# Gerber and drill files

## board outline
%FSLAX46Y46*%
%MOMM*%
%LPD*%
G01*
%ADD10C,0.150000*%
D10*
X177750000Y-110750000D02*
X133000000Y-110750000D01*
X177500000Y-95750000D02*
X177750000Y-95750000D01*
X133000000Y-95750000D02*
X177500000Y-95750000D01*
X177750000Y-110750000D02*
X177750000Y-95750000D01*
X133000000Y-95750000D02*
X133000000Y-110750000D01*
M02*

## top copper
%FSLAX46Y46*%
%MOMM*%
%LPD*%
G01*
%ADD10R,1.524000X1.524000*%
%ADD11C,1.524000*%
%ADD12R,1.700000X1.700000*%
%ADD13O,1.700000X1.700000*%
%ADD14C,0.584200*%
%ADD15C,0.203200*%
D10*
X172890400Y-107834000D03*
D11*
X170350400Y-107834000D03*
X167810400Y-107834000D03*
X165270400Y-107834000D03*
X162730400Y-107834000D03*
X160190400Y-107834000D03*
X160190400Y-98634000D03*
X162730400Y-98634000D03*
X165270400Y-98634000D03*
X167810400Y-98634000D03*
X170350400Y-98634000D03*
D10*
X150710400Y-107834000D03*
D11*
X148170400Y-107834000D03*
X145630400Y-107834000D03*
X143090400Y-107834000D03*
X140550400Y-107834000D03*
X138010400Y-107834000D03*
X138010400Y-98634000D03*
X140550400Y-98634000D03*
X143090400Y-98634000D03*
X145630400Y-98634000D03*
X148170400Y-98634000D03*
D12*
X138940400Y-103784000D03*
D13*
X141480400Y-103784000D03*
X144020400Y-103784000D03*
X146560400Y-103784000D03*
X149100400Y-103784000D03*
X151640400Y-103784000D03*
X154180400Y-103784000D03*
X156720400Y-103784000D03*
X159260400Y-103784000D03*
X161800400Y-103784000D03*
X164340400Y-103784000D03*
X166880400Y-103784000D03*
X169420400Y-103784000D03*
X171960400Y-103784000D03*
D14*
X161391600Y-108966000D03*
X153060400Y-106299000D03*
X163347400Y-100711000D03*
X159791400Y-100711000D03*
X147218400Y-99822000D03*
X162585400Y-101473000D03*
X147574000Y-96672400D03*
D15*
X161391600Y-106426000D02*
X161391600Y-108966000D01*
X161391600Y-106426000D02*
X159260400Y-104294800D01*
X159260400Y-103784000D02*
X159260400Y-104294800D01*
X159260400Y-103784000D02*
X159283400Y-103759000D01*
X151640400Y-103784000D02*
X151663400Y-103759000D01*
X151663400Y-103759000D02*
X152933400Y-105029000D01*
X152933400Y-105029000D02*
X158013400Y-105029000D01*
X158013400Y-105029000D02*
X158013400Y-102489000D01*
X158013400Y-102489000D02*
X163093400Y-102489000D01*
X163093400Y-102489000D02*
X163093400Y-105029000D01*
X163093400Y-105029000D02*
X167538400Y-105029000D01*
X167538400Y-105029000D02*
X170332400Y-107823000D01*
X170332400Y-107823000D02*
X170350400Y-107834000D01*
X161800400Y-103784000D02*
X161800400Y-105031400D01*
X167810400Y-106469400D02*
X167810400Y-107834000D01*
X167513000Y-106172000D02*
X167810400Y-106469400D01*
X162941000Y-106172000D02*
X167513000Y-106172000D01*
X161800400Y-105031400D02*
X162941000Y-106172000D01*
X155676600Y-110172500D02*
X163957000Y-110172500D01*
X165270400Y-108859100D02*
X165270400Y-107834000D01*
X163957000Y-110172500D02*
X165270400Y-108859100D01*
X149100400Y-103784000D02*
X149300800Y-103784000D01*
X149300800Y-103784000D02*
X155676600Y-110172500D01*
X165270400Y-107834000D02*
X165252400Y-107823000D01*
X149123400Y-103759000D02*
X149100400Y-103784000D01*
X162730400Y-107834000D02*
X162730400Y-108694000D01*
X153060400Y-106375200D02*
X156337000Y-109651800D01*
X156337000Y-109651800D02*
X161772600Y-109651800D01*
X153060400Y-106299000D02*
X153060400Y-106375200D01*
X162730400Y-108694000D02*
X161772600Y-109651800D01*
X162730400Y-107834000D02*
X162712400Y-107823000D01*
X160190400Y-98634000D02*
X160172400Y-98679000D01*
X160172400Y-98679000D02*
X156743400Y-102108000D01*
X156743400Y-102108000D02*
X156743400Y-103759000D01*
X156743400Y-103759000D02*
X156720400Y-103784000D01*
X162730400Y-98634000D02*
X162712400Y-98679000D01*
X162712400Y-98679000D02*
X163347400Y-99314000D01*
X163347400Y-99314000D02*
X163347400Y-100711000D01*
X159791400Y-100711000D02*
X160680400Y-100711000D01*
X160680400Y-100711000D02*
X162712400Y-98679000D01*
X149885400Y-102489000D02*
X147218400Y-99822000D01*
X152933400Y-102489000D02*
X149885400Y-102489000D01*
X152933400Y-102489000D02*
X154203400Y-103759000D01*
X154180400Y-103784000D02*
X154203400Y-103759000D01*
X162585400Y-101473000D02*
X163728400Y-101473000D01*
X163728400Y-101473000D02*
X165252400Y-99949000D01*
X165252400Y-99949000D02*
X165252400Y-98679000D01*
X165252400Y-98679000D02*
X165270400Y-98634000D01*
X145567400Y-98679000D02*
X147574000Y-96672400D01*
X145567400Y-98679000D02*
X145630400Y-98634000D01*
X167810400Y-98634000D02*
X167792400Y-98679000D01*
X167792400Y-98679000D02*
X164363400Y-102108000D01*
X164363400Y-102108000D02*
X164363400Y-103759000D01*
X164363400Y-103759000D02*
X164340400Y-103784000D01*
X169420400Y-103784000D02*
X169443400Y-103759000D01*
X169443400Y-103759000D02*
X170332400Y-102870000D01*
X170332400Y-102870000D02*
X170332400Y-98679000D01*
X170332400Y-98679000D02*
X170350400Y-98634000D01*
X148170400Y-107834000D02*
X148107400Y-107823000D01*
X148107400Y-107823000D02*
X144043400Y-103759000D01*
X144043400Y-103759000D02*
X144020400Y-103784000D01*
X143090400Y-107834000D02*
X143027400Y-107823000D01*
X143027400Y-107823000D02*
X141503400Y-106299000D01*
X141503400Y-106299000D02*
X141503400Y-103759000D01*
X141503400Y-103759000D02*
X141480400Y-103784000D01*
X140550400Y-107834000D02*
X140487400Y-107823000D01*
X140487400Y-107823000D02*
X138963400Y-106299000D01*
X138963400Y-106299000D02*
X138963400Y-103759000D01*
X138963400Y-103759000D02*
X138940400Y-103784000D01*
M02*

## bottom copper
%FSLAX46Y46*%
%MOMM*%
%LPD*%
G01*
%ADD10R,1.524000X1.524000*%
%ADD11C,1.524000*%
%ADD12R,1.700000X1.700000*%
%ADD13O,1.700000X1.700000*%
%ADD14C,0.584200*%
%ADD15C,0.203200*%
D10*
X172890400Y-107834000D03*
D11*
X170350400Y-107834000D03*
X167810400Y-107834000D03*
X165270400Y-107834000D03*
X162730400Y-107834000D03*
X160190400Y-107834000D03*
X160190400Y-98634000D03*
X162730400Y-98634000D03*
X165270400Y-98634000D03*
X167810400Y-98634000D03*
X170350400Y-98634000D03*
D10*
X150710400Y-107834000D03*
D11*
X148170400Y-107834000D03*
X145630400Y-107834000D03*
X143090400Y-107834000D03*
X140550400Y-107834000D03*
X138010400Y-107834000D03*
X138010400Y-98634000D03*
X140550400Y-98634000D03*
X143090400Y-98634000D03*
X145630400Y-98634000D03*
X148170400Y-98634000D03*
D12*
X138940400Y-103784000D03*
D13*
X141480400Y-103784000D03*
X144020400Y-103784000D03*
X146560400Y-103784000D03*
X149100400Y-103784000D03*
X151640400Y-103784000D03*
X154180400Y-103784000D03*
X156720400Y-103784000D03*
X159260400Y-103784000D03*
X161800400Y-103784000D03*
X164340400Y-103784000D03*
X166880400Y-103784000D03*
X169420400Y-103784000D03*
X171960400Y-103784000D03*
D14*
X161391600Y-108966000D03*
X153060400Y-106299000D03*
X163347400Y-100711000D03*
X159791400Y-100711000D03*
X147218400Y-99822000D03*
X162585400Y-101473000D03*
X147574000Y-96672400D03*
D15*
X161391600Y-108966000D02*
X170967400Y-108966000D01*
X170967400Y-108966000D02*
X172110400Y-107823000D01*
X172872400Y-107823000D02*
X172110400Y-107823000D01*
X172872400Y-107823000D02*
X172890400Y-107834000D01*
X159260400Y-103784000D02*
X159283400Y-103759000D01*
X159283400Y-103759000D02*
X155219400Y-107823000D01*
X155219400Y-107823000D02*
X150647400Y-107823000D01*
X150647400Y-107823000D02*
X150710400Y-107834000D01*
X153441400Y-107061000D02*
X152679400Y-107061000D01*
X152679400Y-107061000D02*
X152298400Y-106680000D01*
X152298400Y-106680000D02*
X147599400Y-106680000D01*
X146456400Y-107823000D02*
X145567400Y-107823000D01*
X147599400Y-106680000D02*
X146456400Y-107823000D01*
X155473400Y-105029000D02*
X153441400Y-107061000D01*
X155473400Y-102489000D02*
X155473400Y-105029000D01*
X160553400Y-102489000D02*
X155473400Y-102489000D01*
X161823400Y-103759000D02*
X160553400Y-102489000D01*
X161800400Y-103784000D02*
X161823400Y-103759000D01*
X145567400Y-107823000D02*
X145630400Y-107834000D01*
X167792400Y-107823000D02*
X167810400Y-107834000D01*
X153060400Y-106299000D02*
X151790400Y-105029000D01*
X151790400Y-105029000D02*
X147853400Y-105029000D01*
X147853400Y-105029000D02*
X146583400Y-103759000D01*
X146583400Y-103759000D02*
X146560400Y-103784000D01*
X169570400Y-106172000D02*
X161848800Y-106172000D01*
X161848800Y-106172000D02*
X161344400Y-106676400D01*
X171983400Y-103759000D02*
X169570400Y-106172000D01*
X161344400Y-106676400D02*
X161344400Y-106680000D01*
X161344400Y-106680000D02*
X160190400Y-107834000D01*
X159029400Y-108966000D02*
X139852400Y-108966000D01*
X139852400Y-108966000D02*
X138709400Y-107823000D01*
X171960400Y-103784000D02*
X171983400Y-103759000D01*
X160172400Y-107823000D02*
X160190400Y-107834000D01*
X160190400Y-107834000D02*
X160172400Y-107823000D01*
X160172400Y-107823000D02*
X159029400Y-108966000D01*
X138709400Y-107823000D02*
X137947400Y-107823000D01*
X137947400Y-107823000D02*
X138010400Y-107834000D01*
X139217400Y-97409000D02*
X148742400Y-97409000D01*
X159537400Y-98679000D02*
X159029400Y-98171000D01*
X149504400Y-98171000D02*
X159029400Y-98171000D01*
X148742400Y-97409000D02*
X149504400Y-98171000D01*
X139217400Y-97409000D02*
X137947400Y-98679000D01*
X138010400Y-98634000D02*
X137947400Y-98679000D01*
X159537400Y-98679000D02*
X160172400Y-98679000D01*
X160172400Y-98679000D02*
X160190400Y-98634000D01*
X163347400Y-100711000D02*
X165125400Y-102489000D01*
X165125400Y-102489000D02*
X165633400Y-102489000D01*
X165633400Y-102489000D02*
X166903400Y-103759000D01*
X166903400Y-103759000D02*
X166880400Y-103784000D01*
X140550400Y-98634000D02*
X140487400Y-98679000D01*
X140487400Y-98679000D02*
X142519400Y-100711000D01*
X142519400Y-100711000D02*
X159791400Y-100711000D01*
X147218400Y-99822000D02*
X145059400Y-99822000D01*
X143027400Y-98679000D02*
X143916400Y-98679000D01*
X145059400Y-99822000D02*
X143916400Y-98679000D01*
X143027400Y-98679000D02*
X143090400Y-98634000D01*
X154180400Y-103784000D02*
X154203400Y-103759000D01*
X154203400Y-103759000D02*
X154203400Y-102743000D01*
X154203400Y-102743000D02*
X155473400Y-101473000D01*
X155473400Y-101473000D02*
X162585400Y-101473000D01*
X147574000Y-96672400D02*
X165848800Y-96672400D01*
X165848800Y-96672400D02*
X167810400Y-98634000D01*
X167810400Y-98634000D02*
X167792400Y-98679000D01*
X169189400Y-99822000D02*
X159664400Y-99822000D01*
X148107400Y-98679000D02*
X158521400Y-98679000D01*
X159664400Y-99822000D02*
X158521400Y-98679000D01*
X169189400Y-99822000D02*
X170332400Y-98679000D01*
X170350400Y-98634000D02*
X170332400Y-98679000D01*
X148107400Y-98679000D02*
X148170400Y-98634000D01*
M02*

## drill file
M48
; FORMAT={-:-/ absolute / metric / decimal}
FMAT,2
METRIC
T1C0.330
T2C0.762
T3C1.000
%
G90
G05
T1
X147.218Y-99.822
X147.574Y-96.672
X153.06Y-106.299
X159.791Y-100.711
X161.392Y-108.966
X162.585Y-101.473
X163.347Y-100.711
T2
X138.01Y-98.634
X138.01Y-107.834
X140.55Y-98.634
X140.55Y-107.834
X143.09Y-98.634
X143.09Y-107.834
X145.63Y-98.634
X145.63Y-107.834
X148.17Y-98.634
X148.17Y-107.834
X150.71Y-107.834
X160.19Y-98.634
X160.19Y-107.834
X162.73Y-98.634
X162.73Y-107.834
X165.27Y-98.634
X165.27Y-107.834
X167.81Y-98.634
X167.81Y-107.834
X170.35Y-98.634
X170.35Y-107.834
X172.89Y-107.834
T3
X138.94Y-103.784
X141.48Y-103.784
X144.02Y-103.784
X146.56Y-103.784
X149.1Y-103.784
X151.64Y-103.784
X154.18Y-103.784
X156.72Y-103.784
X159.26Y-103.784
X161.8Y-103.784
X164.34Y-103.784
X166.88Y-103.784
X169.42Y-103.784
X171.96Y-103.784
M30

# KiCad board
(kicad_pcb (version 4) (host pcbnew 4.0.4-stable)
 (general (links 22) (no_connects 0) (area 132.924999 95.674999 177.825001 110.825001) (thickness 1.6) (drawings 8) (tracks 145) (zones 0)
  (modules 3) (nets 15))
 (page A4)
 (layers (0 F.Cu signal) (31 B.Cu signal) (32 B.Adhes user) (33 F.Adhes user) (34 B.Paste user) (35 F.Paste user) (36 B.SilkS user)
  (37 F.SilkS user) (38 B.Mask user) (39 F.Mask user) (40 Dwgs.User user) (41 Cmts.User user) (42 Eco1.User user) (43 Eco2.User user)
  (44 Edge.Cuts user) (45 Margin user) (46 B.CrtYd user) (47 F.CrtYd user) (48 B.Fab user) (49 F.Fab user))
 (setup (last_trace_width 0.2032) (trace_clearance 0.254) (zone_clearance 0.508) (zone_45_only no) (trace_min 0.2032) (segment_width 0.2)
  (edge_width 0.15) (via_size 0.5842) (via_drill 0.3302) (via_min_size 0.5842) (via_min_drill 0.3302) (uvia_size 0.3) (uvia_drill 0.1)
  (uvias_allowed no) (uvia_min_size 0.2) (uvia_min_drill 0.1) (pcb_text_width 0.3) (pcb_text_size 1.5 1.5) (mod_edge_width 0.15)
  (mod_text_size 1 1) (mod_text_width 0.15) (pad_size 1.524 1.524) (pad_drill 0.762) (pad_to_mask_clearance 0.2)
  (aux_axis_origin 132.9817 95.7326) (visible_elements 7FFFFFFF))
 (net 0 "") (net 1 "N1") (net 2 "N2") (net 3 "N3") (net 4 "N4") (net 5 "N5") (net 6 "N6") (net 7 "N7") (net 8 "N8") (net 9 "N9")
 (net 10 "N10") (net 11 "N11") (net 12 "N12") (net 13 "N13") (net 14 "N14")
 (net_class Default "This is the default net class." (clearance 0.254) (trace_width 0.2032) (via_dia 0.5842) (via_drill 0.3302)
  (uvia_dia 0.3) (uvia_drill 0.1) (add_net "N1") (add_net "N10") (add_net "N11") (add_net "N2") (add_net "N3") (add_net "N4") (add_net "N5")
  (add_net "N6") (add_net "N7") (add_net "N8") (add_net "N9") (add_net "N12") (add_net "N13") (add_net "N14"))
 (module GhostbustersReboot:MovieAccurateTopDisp (layer B.Cu) (at 166.5404 103.234 180)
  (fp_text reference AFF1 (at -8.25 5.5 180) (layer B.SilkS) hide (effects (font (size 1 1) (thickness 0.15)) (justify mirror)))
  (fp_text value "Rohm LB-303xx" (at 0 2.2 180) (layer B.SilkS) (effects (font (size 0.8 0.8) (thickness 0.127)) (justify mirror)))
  (pad 1 thru_hole rect (at -6.35 -4.6 180) (size 1.524 1.524) (drill 0.762) (layers *.Cu *.Mask) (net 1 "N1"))
  (pad 2 thru_hole circle (at -3.81 -4.6 180) (size 1.524 1.524) (drill 0.762) (layers *.Cu *.Mask) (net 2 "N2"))
  (pad 3 thru_hole circle (at -1.27 -4.6 180) (size 1.524 1.524) (drill 0.762) (layers *.Cu *.Mask) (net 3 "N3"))
  (pad 4 thru_hole circle (at 1.27 -4.6 180) (size 1.524 1.524) (drill 0.762) (layers *.Cu *.Mask) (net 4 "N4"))
  (pad 5 thru_hole circle (at 3.81 -4.6 180) (size 1.524 1.524) (drill 0.762) (layers *.Cu *.Mask) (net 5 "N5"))
  (pad 6 thru_hole circle (at 6.35 -4.6 180) (size 1.524 1.524) (drill 0.762) (layers *.Cu *.Mask) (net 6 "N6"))
  (pad 7 thru_hole circle (at 6.35 4.6 180) (size 1.524 1.524) (drill 0.762) (layers *.Cu *.Mask) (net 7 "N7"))
  (pad 8 thru_hole circle (at 3.81 4.6 180) (size 1.524 1.524) (drill 0.762) (layers *.Cu *.Mask) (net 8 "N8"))
  (pad 9 thru_hole circle (at 1.27 4.6 180) (size 1.524 1.524) (drill 0.762) (layers *.Cu *.Mask) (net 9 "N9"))
  (pad 10 thru_hole circle (at -1.27 4.6 180) (size 1.524 1.524) (drill 0.762) (layers *.Cu *.Mask) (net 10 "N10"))
  (pad 11 thru_hole circle (at -3.81 4.6 180) (size 1.524 1.524) (drill 0.762) (layers *.Cu *.Mask) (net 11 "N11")))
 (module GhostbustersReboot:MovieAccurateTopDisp (layer B.Cu) (at 144.3604 103.234 180)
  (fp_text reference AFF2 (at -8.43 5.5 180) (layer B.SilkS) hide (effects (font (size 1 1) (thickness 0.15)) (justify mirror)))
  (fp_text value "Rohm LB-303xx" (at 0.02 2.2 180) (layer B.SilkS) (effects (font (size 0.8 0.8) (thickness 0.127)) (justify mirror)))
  (pad 1 thru_hole rect (at -6.35 -4.6 180) (size 1.524 1.524) (drill 0.762) (layers *.Cu *.Mask) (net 1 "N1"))
  (pad 2 thru_hole circle (at -3.81 -4.6 180) (size 1.524 1.524) (drill 0.762) (layers *.Cu *.Mask) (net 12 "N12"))
  (pad 3 thru_hole circle (at -1.27 -4.6 180) (size 1.524 1.524) (drill 0.762) (layers *.Cu *.Mask) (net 3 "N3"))
  (pad 4 thru_hole circle (at 1.27 -4.6 180) (size 1.524 1.524) (drill 0.762) (layers *.Cu *.Mask) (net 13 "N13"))
  (pad 5 thru_hole circle (at 3.81 -4.6 180) (size 1.524 1.524) (drill 0.762) (layers *.Cu *.Mask) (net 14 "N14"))
  (pad 6 thru_hole circle (at 6.35 -4.6 180) (size 1.524 1.524) (drill 0.762) (layers *.Cu *.Mask) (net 6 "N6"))
  (pad 7 thru_hole circle (at 6.35 4.6 180) (size 1.524 1.524) (drill 0.762) (layers *.Cu *.Mask) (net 7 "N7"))
  (pad 8 thru_hole circle (at 3.81 4.6 180) (size 1.524 1.524) (drill 0.762) (layers *.Cu *.Mask) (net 8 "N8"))
  (pad 9 thru_hole circle (at 1.27 4.6 180) (size 1.524 1.524) (drill 0.762) (layers *.Cu *.Mask) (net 9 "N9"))
  (pad 10 thru_hole circle (at -1.27 4.6 180) (size 1.524 1.524) (drill 0.762) (layers *.Cu *.Mask) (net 10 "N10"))
  (pad 11 thru_hole circle (at -3.81 4.6 180) (size 1.524 1.524) (drill 0.762) (layers *.Cu *.Mask) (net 11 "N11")))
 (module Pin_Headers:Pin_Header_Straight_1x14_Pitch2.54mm (layer F.Cu) (at 138.9404 103.784 90)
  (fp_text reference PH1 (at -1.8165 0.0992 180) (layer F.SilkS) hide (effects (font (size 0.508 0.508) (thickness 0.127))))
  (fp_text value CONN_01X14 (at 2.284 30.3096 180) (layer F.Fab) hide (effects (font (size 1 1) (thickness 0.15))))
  (pad 1 thru_hole rect (at 0 0 90) (size 1.7 1.7) (drill 1) (layers *.Cu *.Mask) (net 14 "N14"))
  (pad 2 thru_hole oval (at 0 2.54 90) (size 1.7 1.7) (drill 1) (layers *.Cu *.Mask) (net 13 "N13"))
  (pad 3 thru_hole oval (at 0 5.08 90) (size 1.7 1.7) (drill 1) (layers *.Cu *.Mask) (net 12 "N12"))
  (pad 4 thru_hole oval (at 0 7.62 90) (size 1.7 1.7) (drill 1) (layers *.Cu *.Mask) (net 5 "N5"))
  (pad 5 thru_hole oval (at 0 10.16 90) (size 1.7 1.7) (drill 1) (layers *.Cu *.Mask) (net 4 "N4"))
  (pad 6 thru_hole oval (at 0 12.7 90) (size 1.7 1.7) (drill 1) (layers *.Cu *.Mask) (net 2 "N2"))
  (pad 7 thru_hole oval (at 0 15.24 90) (size 1.7 1.7) (drill 1) (layers *.Cu *.Mask) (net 9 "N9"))
  (pad 8 thru_hole oval (at 0 17.78 90) (size 1.7 1.7) (drill 1) (layers *.Cu *.Mask) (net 7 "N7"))
  (pad 9 thru_hole oval (at 0 20.32 90) (size 1.7 1.7) (drill 1) (layers *.Cu *.Mask) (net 1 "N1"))
  (pad 10 thru_hole oval (at 0 22.86 90) (size 1.7 1.7) (drill 1) (layers *.Cu *.Mask) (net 3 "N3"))
  (pad 11 thru_hole oval (at 0 25.4 90) (size 1.7 1.7) (drill 1) (layers *.Cu *.Mask) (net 10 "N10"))
  (pad 12 thru_hole oval (at 0 27.94 90) (size 1.7 1.7) (drill 1) (layers *.Cu *.Mask) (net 8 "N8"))
  (pad 13 thru_hole oval (at 0 30.48 90) (size 1.7 1.7) (drill 1) (layers *.Cu *.Mask) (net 11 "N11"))
  (pad 14 thru_hole oval (at 0 33.02 90) (size 1.7 1.7) (drill 1) (layers *.Cu *.Mask) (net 6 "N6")))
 (gr_line (start 177.75 110.75) (end 133 110.75) (angle 90) (layer Edge.Cuts) (width 0.15))
 (gr_line (start 177.5 95.75) (end 177.75 95.75) (angle 90) (layer Edge.Cuts) (width 0.15))
 (gr_line (start 133 95.75) (end 177.5 95.75) (angle 90) (layer Edge.Cuts) (width 0.15))
 (gr_line (start 177.75 110.75) (end 177.75 95.75) (angle 90) (layer Edge.Cuts) (width 0.15))
 (gr_line (start 133 95.75) (end 133 110.75) (angle 90) (layer Edge.Cuts) (width 0.15))
 (segment (start 161.3916 108.966) (end 170.9674 108.966) (width 0.2032) (layer B.Cu) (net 1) (status 80000))
 (segment (start 170.9674 108.966) (end 172.1104 107.823) (width 0.2032) (layer B.Cu) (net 1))
 (segment (start 172.8724 107.823) (end 172.1104 107.823) (width 0.2032) (layer B.Cu) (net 1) (status 80010))
 (via (at 161.3916 108.966) (size 0.5842) (layers F.Cu B.Cu) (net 1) (status 80000))
 (segment (start 161.3916 106.426) (end 161.3916 108.966) (width 0.2032) (layer F.Cu) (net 1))
 (segment (start 161.3916 106.426) (end 159.2604 104.2948) (width 0.2032) (layer F.Cu) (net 1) (status 20))
 (segment (start 159.2604 103.784) (end 159.2604 104.2948) (width 0.2032) (layer F.Cu) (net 1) (status 30))
 (segment (start 159.2604 103.784) (end 159.2834 103.759) (width 0.2032) (layer F.Cu) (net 1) (status 80030))
 (segment (start 172.8724 107.823) (end 172.8904 107.834) (width 0.2032) (layer B.Cu) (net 1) (status 80030))
 (segment (start 159.2604 103.784) (end 159.2834 103.759) (width 0.2032) (layer B.Cu) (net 1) (status 80030))
 (segment (start 159.2834 103.759) (end 155.2194 107.823) (width 0.2032) (layer B.Cu) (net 1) (status 80010))
 (segment (start 155.2194 107.823) (end 150.6474 107.823) (width 0.2032) (layer B.Cu) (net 1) (status 80020))
 (segment (start 150.6474 107.823) (end 150.7104 107.834) (width 0.2032) (layer B.Cu) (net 1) (status 80030))
 (segment (start 151.6404 103.784) (end 151.6634 103.759) (width 0.2032) (layer F.Cu) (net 2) (status 80030))
 (segment (start 151.6634 103.759) (end 152.9334 105.029) (width 0.2032) (layer F.Cu) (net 2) (status 80010))
 (segment (start 152.9334 105.029) (end 158.0134 105.029) (width 0.2032) (layer F.Cu) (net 2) (status 80000))
 (segment (start 158.0134 105.029) (end 158.0134 102.489) (width 0.2032) (layer F.Cu) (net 2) (status 80000))
 (segment (start 158.0134 102.489) (end 163.0934 102.489) (width 0.2032) (layer F.Cu) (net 2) (status 80000))
 (segment (start 163.0934 102.489) (end 163.0934 105.029) (width 0.2032) (layer F.Cu) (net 2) (status 80000))
 (segment (start 163.0934 105.029) (end 167.5384 105.029) (width 0.2032) (layer F.Cu) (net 2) (status 80000))
 (segment (start 167.5384 105.029) (end 170.3324 107.823) (width 0.2032) (layer F.Cu) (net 2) (status 80020))
 (segment (start 170.3324 107.823) (end 170.3504 107.834) (width 0.2032) (layer F.Cu) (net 2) (status 80030))
 (segment (start 161.8004 103.784) (end 161.8004 105.0314) (width 0.2032) (layer F.Cu) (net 3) (status 10))
 (segment (start 167.8104 106.4694) (end 167.8104 107.834) (width 0.2032) (layer F.Cu) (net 3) (status 20))
 (segment (start 167.513 106.172) (end 167.8104 106.4694) (width 0.2032) (layer F.Cu) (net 3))
 (segment (start 162.941 106.172) (end 167.513 106.172) (width 0.2032) (layer F.Cu) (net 3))
 (segment (start 161.8004 105.0314) (end 162.941 106.172) (width 0.2032) (layer F.Cu) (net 3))
 (segment (start 153.4414 107.061) (end 152.6794 107.061) (width 0.2032) (layer B.Cu) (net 3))
 (segment (start 152.6794 107.061) (end 152.2984 106.68) (width 0.2032) (layer B.Cu) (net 3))
 (segment (start 152.2984 106.68) (end 147.5994 106.68) (width 0.2032) (layer B.Cu) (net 3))
 (segment (start 146.4564 107.823) (end 145.5674 107.823) (width 0.2032) (layer B.Cu) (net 3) (status 80020))
 (segment (start 147.5994 106.68) (end 146.4564 107.823) (width 0.2032) (layer B.Cu) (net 3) (status 80000))
 (segment (start 155.4734 105.029) (end 153.4414 107.061) (width 0.2032) (layer B.Cu) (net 3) (status 80000))
 (segment (start 155.4734 102.489) (end 155.4734 105.029) (width 0.2032) (layer B.Cu) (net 3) (status 80000))
 (segment (start 160.5534 102.489) (end 155.4734 102.489) (width 0.2032) (layer B.Cu) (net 3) (status 80000))
 (segment (start 161.8234 103.759) (end 160.5534 102.489) (width 0.2032) (layer B.Cu) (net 3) (status 80010))
 (segment (start 161.8004 103.784) (end 161.8234 103.759) (width 0.2032) (layer B.Cu) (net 3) (status 80030))
 (segment (start 145.5674 107.823) (end 145.6304 107.834) (width 0.2032) (layer B.Cu) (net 3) (status 80030))
 (segment (start 167.7924 107.823) (end 167.8104 107.834) (width 0.2032) (layer B.Cu) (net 3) (status 80030))
 (segment (start 155.6766 110.1725) (end 163.957 110.1725) (width 0.2032) (layer F.Cu) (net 4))
 (segment (start 165.2704 108.8591) (end 165.2704 107.834) (width 0.2032) (layer F.Cu) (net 4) (status 20))
 (segment (start 163.957 110.1725) (end 165.2704 108.8591) (width 0.2032) (layer F.Cu) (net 4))
 (segment (start 149.1004 103.784) (end 149.3008 103.784) (width 0.2032) (layer F.Cu) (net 4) (status 30))
 (segment (start 149.3008 103.784) (end 155.6766 110.1725) (width 0.2032) (layer F.Cu) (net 4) (status 10))
 (segment (start 165.2704 107.834) (end 165.2524 107.823) (width 0.2032) (layer F.Cu) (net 4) (status 80030))
 (segment (start 149.1234 103.759) (end 149.1004 103.784) (width 0.2032) (layer F.Cu) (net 4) (status 80030))
 (segment (start 162.7304 107.834) (end 162.7304 108.694) (width 0.2032) (layer F.Cu) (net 5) (status 10))
 (segment (start 153.0604 106.3752) (end 156.337 109.6518) (width 0.2032) (layer F.Cu) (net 5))
 (segment (start 156.337 109.6518) (end 161.7726 109.6518) (width 0.2032) (layer F.Cu) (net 5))
 (via (at 153.0604 106.299) (size 0.5842) (layers F.Cu B.Cu) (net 5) (status 80000))
 (segment (start 153.0604 106.299) (end 151.7904 105.029) (width 0.2032) (layer B.Cu) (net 5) (status 80000))
 (segment (start 151.7904 105.029) (end 147.8534 105.029) (width 0.2032) (layer B.Cu) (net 5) (status 80000))
 (segment (start 147.8534 105.029) (end 146.5834 103.759) (width 0.2032) (layer B.Cu) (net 5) (status 80020))
 (segment (start 153.0604 106.299) (end 153.0604 106.3752) (width 0.2032) (layer F.Cu) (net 5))
 (segment (start 162.7304 108.694) (end 161.7726 109.6518) (width 0.2032) (layer F.Cu) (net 5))
 (segment (start 162.7304 107.834) (end 162.7124 107.823) (width 0.2032) (layer F.Cu) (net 5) (status 80030))
 (segment (start 146.5834 103.759) (end 146.5604 103.784) (width 0.2032) (layer B.Cu) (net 5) (status 80030))
 (segment (start 169.5704 106.172) (end 161.8488 106.172) (width 0.2032) (layer B.Cu) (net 6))
 (segment (start 161.8488 106.172) (end 161.3444 106.6764) (width 0.2032) (layer B.Cu) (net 6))
 (segment (start 171.9834 103.759) (end 169.5704 106.172) (width 0.2032) (layer B.Cu) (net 6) (status 80010))
 (segment (start 161.3444 106.6764) (end 161.3444 106.68) (width 0.2032) (layer B.Cu) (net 6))
 (segment (start 161.3444 106.68) (end 160.1904 107.834) (width 0.2032) (layer B.Cu) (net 6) (status 20))
 (segment (start 159.0294 108.966) (end 139.8524 108.966) (width 0.2032) (layer B.Cu) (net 6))
 (segment (start 139.8524 108.966) (end 138.7094 107.823) (width 0.2032) (layer B.Cu) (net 6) (status 80020))
 (segment (start 171.9604 103.784) (end 171.9834 103.759) (width 0.2032) (layer B.Cu) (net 6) (status 80030))
 (segment (start 160.1724 107.823) (end 160.1904 107.834) (width 0.2032) (layer B.Cu) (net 6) (status 80030))
 (segment (start 160.1904 107.834) (end 160.1724 107.823) (width 0.2032) (layer B.Cu) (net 6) (status 80030))
 (segment (start 160.1724 107.823) (end 159.0294 108.966) (width 0.2032) (layer B.Cu) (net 6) (status 80010))
 (segment (start 138.7094 107.823) (end 137.9474 107.823) (width 0.2032) (layer B.Cu) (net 6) (status 80030))
 (segment (start 137.9474 107.823) (end 138.0104 107.834) (width 0.2032) (layer B.Cu) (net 6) (status 80030))
 (segment (start 139.2174 97.409) (end 148.7424 97.409) (width 0.2032) (layer B.Cu) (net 7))
 (segment (start 159.5374 98.679) (end 159.0294 98.171) (width 0.2032) (layer B.Cu) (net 7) (status 80010))
 (segment (start 149.5044 98.171) (end 159.0294 98.171) (width 0.2032) (layer B.Cu) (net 7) (status 80000))
 (segment (start 148.7424 97.409) (end 149.5044 98.171) (width 0.2032) (layer B.Cu) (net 7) (status 80000))
 (segment (start 139.2174 97.409) (end 137.9474 98.679) (width 0.2032) (layer B.Cu) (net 7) (status 80020))
 (segment (start 138.0104 98.634) (end 137.9474 98.679) (width 0.2032) (layer B.Cu) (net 7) (status 80030))
 (segment (start 159.5374 98.679) (end 160.1724 98.679) (width 0.2032) (layer B.Cu) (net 7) (status 80030))
 (segment (start 160.1724 98.679) (end 160.1904 98.634) (width 0.2032) (layer B.Cu) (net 7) (status 80030))
 (segment (start 160.1904 98.634) (end 160.1724 98.679) (width 0.2032) (layer F.Cu) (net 7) (status 80030))
 (segment (start 160.1724 98.679) (end 156.7434 102.108) (width 0.2032) (layer F.Cu) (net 7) (status 80010))
 (segment (start 156.7434 102.108) (end 156.7434 103.759) (width 0.2032) (layer F.Cu) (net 7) (status 80020))
 (segment (start 156.7434 103.759) (end 156.7204 103.784) (width 0.2032) (layer F.Cu) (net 7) (status 80030))
 (segment (start 162.7304 98.634) (end 162.7124 98.679) (width 0.2032) (layer F.Cu) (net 8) (status 80030))
 (segment (start 162.7124 98.679) (end 163.3474 99.314) (width 0.2032) (layer F.Cu) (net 8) (status 80010))
 (segment (start 163.3474 99.314) (end 163.3474 100.711) (width 0.2032) (layer F.Cu) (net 8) (status 80000))
 (via (at 163.3474 100.711) (size 0.5842) (layers F.Cu B.Cu) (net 8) (status 80000))
 (segment (start 163.3474 100.711) (end 165.1254 102.489) (width 0.2032) (layer B.Cu) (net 8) (status 80000))
 (segment (start 165.1254 102.489) (end 165.6334 102.489) (width 0.2032) (layer B.Cu) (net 8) (status 80000))
 (segment (start 165.6334 102.489) (end 166.9034 103.759) (width 0.2032) (layer B.Cu) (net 8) (status 80020))
 (segment (start 166.9034 103.759) (end 166.8804 103.784) (width 0.2032) (layer B.Cu) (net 8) (status 80030))
 (segment (start 140.5504 98.634) (end 140.4874 98.679) (width 0.2032) (layer B.Cu) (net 8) (status 80030))
 (segment (start 140.4874 98.679) (end 142.5194 100.711) (width 0.2032) (layer B.Cu) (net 8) (status 80010))
 (segment (start 142.5194 100.711) (end 159.7914 100.711) (width 0.2032) (layer B.Cu) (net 8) (status 80000))
 (via (at 159.7914 100.711) (size 0.5842) (layers F.Cu B.Cu) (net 8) (status 80000))
 (segment (start 159.7914 100.711) (end 160.6804 100.711) (width 0.2032) (layer F.Cu) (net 8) (status 80000))
 (segment (start 160.6804 100.711) (end 162.7124 98.679) (width 0.2032) (layer F.Cu) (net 8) (status 80020))
 (segment (start 147.2184 99.822) (end 145.0594 99.822) (width 0.2032) (layer B.Cu) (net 9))
 (segment (start 143.0274 98.679) (end 143.9164 98.679) (width 0.2032) (layer B.Cu) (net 9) (status 80010))
 (segment (start 145.0594 99.822) (end 143.9164 98.679) (width 0.2032) (layer B.Cu) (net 9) (status 80000))
 (via (at 147.2184 99.822) (size 0.5842) (layers F.Cu B.Cu) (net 9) (status 80000))
 (segment (start 149.8854 102.489) (end 147.2184 99.822) (width 0.2032) (layer F.Cu) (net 9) (status 80000))
 (segment (start 152.9334 102.489) (end 149.8854 102.489) (width 0.2032) (layer F.Cu) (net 9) (status 80000))
 (segment (start 152.9334 102.489) (end 154.2034 103.759) (width 0.2032) (layer F.Cu) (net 9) (status 80020))
 (segment (start 154.1804 103.784) (end 154.2034 103.759) (width 0.2032) (layer F.Cu) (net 9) (status 80030))
 (segment (start 143.0274 98.679) (end 143.0904 98.634) (width 0.2032) (layer B.Cu) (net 9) (status 80030))
 (segment (start 154.1804 103.784) (end 154.2034 103.759) (width 0.2032) (layer B.Cu) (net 9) (status 80030))
 (segment (start 154.2034 103.759) (end 154.2034 102.743) (width 0.2032) (layer B.Cu) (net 9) (status 80010))
 (segment (start 154.2034 102.743) (end 155.4734 101.473) (width 0.2032) (layer B.Cu) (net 9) (status 80000))
 (segment (start 155.4734 101.473) (end 162.5854 101.473) (width 0.2032) (layer B.Cu) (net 9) (status 80000))
 (via (at 162.5854 101.473) (size 0.5842) (layers F.Cu B.Cu) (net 9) (status 80000))
 (segment (start 162.5854 101.473) (end 163.7284 101.473) (width 0.2032) (layer F.Cu) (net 9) (status 80000))
 (segment (start 163.7284 101.473) (end 165.2524 99.949) (width 0.2032) (layer F.Cu) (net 9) (status 80000))
 (segment (start 165.2524 99.949) (end 165.2524 98.679) (width 0.2032) (layer F.Cu) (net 9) (status 80020))
 (segment (start 165.2524 98.679) (end 165.2704 98.634) (width 0.2032) (layer F.Cu) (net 9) (status 80030))
 (segment (start 147.574 96.6724) (end 165.8488 96.6724) (width 0.2032) (layer B.Cu) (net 10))
 (segment (start 145.5674 98.679) (end 147.574 96.6724) (width 0.2032) (layer F.Cu) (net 10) (status 80010))
 (via (at 147.574 96.6724) (size 0.5842) (layers F.Cu B.Cu) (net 10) (status 80000))
 (segment (start 165.8488 96.6724) (end 167.8104 98.634) (width 0.2032) (layer B.Cu) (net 10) (status 20))
 (segment (start 167.8104 98.634) (end 167.7924 98.679) (width 0.2032) (layer B.Cu) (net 10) (status 80030))
 (segment (start 145.5674 98.679) (end 145.6304 98.634) (width 0.2032) (layer F.Cu) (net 10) (status 80030))
 (segment (start 167.8104 98.634) (end 167.7924 98.679) (width 0.2032) (layer F.Cu) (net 10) (status 80030))
 (segment (start 167.7924 98.679) (end 164.3634 102.108) (width 0.2032) (layer F.Cu) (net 10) (status 80010))
 (segment (start 164.3634 102.108) (end 164.3634 103.759) (width 0.2032) (layer F.Cu) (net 10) (status 80020))
 (segment (start 164.3634 103.759) (end 164.3404 103.784) (width 0.2032) (layer F.Cu) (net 10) (status 80030))
 (segment (start 169.1894 99.822) (end 159.6644 99.822) (width 0.2032) (layer B.Cu) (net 11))
 (segment (start 148.1074 98.679) (end 158.5214 98.679) (width 0.2032) (layer B.Cu) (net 11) (status 80010))
 (segment (start 159.6644 99.822) (end 158.5214 98.679) (width 0.2032) (layer B.Cu) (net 11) (status 80000))
 (segment (start 169.1894 99.822) (end 170.3324 98.679) (width 0.2032) (layer B.Cu) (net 11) (status 80020))
 (segment (start 170.3504 98.634) (end 170.3324 98.679) (width 0.2032) (layer B.Cu) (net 11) (status 80030))
 (segment (start 148.1074 98.679) (end 148.1704 98.634) (width 0.2032) (layer B.Cu) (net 11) (status 80030))
 (segment (start 169.4204 103.784) (end 169.4434 103.759) (width 0.2032) (layer F.Cu) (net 11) (status 80030))
 (segment (start 169.4434 103.759) (end 170.3324 102.87) (width 0.2032) (layer F.Cu) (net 11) (status 80010))
 (segment (start 170.3324 102.87) (end 170.3324 98.679) (width 0.2032) (layer F.Cu) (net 11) (status 80020))
 (segment (start 170.3324 98.679) (end 170.3504 98.634) (width 0.2032) (layer F.Cu) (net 11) (status 80030))
 (segment (start 148.1704 107.834) (end 148.1074 107.823) (width 0.2032) (layer F.Cu) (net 12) (status 80030))
 (segment (start 148.1074 107.823) (end 144.0434 103.759) (width 0.2032) (layer F.Cu) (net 12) (status 80030))
 (segment (start 144.0434 103.759) (end 144.0204 103.784) (width 0.2032) (layer F.Cu) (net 12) (status 80030))
 (segment (start 143.0904 107.834) (end 143.0274 107.823) (width 0.2032) (layer F.Cu) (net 13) (status 80030))
 (segment (start 143.0274 107.823) (end 141.5034 106.299) (width 0.2032) (layer F.Cu) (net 13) (status 80010))
 (segment (start 141.5034 106.299) (end 141.5034 103.759) (width 0.2032) (layer F.Cu) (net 13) (status 80020))
 (segment (start 141.5034 103.759) (end 141.4804 103.784) (width 0.2032) (layer F.Cu) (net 13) (status 80030))
 (segment (start 140.5504 107.834) (end 140.4874 107.823) (width 0.2032) (layer F.Cu) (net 14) (status 80030))
 (segment (start 140.4874 107.823) (end 138.9634 106.299) (width 0.2032) (layer F.Cu) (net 14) (status 80010))
 (segment (start 138.9634 106.299) (end 138.9634 103.759) (width 0.2032) (layer F.Cu) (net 14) (status 80020))
 (segment (start 138.9634 103.759) (end 138.9404 103.784) (width 0.2032) (layer F.Cu) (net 14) (status 80030)))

